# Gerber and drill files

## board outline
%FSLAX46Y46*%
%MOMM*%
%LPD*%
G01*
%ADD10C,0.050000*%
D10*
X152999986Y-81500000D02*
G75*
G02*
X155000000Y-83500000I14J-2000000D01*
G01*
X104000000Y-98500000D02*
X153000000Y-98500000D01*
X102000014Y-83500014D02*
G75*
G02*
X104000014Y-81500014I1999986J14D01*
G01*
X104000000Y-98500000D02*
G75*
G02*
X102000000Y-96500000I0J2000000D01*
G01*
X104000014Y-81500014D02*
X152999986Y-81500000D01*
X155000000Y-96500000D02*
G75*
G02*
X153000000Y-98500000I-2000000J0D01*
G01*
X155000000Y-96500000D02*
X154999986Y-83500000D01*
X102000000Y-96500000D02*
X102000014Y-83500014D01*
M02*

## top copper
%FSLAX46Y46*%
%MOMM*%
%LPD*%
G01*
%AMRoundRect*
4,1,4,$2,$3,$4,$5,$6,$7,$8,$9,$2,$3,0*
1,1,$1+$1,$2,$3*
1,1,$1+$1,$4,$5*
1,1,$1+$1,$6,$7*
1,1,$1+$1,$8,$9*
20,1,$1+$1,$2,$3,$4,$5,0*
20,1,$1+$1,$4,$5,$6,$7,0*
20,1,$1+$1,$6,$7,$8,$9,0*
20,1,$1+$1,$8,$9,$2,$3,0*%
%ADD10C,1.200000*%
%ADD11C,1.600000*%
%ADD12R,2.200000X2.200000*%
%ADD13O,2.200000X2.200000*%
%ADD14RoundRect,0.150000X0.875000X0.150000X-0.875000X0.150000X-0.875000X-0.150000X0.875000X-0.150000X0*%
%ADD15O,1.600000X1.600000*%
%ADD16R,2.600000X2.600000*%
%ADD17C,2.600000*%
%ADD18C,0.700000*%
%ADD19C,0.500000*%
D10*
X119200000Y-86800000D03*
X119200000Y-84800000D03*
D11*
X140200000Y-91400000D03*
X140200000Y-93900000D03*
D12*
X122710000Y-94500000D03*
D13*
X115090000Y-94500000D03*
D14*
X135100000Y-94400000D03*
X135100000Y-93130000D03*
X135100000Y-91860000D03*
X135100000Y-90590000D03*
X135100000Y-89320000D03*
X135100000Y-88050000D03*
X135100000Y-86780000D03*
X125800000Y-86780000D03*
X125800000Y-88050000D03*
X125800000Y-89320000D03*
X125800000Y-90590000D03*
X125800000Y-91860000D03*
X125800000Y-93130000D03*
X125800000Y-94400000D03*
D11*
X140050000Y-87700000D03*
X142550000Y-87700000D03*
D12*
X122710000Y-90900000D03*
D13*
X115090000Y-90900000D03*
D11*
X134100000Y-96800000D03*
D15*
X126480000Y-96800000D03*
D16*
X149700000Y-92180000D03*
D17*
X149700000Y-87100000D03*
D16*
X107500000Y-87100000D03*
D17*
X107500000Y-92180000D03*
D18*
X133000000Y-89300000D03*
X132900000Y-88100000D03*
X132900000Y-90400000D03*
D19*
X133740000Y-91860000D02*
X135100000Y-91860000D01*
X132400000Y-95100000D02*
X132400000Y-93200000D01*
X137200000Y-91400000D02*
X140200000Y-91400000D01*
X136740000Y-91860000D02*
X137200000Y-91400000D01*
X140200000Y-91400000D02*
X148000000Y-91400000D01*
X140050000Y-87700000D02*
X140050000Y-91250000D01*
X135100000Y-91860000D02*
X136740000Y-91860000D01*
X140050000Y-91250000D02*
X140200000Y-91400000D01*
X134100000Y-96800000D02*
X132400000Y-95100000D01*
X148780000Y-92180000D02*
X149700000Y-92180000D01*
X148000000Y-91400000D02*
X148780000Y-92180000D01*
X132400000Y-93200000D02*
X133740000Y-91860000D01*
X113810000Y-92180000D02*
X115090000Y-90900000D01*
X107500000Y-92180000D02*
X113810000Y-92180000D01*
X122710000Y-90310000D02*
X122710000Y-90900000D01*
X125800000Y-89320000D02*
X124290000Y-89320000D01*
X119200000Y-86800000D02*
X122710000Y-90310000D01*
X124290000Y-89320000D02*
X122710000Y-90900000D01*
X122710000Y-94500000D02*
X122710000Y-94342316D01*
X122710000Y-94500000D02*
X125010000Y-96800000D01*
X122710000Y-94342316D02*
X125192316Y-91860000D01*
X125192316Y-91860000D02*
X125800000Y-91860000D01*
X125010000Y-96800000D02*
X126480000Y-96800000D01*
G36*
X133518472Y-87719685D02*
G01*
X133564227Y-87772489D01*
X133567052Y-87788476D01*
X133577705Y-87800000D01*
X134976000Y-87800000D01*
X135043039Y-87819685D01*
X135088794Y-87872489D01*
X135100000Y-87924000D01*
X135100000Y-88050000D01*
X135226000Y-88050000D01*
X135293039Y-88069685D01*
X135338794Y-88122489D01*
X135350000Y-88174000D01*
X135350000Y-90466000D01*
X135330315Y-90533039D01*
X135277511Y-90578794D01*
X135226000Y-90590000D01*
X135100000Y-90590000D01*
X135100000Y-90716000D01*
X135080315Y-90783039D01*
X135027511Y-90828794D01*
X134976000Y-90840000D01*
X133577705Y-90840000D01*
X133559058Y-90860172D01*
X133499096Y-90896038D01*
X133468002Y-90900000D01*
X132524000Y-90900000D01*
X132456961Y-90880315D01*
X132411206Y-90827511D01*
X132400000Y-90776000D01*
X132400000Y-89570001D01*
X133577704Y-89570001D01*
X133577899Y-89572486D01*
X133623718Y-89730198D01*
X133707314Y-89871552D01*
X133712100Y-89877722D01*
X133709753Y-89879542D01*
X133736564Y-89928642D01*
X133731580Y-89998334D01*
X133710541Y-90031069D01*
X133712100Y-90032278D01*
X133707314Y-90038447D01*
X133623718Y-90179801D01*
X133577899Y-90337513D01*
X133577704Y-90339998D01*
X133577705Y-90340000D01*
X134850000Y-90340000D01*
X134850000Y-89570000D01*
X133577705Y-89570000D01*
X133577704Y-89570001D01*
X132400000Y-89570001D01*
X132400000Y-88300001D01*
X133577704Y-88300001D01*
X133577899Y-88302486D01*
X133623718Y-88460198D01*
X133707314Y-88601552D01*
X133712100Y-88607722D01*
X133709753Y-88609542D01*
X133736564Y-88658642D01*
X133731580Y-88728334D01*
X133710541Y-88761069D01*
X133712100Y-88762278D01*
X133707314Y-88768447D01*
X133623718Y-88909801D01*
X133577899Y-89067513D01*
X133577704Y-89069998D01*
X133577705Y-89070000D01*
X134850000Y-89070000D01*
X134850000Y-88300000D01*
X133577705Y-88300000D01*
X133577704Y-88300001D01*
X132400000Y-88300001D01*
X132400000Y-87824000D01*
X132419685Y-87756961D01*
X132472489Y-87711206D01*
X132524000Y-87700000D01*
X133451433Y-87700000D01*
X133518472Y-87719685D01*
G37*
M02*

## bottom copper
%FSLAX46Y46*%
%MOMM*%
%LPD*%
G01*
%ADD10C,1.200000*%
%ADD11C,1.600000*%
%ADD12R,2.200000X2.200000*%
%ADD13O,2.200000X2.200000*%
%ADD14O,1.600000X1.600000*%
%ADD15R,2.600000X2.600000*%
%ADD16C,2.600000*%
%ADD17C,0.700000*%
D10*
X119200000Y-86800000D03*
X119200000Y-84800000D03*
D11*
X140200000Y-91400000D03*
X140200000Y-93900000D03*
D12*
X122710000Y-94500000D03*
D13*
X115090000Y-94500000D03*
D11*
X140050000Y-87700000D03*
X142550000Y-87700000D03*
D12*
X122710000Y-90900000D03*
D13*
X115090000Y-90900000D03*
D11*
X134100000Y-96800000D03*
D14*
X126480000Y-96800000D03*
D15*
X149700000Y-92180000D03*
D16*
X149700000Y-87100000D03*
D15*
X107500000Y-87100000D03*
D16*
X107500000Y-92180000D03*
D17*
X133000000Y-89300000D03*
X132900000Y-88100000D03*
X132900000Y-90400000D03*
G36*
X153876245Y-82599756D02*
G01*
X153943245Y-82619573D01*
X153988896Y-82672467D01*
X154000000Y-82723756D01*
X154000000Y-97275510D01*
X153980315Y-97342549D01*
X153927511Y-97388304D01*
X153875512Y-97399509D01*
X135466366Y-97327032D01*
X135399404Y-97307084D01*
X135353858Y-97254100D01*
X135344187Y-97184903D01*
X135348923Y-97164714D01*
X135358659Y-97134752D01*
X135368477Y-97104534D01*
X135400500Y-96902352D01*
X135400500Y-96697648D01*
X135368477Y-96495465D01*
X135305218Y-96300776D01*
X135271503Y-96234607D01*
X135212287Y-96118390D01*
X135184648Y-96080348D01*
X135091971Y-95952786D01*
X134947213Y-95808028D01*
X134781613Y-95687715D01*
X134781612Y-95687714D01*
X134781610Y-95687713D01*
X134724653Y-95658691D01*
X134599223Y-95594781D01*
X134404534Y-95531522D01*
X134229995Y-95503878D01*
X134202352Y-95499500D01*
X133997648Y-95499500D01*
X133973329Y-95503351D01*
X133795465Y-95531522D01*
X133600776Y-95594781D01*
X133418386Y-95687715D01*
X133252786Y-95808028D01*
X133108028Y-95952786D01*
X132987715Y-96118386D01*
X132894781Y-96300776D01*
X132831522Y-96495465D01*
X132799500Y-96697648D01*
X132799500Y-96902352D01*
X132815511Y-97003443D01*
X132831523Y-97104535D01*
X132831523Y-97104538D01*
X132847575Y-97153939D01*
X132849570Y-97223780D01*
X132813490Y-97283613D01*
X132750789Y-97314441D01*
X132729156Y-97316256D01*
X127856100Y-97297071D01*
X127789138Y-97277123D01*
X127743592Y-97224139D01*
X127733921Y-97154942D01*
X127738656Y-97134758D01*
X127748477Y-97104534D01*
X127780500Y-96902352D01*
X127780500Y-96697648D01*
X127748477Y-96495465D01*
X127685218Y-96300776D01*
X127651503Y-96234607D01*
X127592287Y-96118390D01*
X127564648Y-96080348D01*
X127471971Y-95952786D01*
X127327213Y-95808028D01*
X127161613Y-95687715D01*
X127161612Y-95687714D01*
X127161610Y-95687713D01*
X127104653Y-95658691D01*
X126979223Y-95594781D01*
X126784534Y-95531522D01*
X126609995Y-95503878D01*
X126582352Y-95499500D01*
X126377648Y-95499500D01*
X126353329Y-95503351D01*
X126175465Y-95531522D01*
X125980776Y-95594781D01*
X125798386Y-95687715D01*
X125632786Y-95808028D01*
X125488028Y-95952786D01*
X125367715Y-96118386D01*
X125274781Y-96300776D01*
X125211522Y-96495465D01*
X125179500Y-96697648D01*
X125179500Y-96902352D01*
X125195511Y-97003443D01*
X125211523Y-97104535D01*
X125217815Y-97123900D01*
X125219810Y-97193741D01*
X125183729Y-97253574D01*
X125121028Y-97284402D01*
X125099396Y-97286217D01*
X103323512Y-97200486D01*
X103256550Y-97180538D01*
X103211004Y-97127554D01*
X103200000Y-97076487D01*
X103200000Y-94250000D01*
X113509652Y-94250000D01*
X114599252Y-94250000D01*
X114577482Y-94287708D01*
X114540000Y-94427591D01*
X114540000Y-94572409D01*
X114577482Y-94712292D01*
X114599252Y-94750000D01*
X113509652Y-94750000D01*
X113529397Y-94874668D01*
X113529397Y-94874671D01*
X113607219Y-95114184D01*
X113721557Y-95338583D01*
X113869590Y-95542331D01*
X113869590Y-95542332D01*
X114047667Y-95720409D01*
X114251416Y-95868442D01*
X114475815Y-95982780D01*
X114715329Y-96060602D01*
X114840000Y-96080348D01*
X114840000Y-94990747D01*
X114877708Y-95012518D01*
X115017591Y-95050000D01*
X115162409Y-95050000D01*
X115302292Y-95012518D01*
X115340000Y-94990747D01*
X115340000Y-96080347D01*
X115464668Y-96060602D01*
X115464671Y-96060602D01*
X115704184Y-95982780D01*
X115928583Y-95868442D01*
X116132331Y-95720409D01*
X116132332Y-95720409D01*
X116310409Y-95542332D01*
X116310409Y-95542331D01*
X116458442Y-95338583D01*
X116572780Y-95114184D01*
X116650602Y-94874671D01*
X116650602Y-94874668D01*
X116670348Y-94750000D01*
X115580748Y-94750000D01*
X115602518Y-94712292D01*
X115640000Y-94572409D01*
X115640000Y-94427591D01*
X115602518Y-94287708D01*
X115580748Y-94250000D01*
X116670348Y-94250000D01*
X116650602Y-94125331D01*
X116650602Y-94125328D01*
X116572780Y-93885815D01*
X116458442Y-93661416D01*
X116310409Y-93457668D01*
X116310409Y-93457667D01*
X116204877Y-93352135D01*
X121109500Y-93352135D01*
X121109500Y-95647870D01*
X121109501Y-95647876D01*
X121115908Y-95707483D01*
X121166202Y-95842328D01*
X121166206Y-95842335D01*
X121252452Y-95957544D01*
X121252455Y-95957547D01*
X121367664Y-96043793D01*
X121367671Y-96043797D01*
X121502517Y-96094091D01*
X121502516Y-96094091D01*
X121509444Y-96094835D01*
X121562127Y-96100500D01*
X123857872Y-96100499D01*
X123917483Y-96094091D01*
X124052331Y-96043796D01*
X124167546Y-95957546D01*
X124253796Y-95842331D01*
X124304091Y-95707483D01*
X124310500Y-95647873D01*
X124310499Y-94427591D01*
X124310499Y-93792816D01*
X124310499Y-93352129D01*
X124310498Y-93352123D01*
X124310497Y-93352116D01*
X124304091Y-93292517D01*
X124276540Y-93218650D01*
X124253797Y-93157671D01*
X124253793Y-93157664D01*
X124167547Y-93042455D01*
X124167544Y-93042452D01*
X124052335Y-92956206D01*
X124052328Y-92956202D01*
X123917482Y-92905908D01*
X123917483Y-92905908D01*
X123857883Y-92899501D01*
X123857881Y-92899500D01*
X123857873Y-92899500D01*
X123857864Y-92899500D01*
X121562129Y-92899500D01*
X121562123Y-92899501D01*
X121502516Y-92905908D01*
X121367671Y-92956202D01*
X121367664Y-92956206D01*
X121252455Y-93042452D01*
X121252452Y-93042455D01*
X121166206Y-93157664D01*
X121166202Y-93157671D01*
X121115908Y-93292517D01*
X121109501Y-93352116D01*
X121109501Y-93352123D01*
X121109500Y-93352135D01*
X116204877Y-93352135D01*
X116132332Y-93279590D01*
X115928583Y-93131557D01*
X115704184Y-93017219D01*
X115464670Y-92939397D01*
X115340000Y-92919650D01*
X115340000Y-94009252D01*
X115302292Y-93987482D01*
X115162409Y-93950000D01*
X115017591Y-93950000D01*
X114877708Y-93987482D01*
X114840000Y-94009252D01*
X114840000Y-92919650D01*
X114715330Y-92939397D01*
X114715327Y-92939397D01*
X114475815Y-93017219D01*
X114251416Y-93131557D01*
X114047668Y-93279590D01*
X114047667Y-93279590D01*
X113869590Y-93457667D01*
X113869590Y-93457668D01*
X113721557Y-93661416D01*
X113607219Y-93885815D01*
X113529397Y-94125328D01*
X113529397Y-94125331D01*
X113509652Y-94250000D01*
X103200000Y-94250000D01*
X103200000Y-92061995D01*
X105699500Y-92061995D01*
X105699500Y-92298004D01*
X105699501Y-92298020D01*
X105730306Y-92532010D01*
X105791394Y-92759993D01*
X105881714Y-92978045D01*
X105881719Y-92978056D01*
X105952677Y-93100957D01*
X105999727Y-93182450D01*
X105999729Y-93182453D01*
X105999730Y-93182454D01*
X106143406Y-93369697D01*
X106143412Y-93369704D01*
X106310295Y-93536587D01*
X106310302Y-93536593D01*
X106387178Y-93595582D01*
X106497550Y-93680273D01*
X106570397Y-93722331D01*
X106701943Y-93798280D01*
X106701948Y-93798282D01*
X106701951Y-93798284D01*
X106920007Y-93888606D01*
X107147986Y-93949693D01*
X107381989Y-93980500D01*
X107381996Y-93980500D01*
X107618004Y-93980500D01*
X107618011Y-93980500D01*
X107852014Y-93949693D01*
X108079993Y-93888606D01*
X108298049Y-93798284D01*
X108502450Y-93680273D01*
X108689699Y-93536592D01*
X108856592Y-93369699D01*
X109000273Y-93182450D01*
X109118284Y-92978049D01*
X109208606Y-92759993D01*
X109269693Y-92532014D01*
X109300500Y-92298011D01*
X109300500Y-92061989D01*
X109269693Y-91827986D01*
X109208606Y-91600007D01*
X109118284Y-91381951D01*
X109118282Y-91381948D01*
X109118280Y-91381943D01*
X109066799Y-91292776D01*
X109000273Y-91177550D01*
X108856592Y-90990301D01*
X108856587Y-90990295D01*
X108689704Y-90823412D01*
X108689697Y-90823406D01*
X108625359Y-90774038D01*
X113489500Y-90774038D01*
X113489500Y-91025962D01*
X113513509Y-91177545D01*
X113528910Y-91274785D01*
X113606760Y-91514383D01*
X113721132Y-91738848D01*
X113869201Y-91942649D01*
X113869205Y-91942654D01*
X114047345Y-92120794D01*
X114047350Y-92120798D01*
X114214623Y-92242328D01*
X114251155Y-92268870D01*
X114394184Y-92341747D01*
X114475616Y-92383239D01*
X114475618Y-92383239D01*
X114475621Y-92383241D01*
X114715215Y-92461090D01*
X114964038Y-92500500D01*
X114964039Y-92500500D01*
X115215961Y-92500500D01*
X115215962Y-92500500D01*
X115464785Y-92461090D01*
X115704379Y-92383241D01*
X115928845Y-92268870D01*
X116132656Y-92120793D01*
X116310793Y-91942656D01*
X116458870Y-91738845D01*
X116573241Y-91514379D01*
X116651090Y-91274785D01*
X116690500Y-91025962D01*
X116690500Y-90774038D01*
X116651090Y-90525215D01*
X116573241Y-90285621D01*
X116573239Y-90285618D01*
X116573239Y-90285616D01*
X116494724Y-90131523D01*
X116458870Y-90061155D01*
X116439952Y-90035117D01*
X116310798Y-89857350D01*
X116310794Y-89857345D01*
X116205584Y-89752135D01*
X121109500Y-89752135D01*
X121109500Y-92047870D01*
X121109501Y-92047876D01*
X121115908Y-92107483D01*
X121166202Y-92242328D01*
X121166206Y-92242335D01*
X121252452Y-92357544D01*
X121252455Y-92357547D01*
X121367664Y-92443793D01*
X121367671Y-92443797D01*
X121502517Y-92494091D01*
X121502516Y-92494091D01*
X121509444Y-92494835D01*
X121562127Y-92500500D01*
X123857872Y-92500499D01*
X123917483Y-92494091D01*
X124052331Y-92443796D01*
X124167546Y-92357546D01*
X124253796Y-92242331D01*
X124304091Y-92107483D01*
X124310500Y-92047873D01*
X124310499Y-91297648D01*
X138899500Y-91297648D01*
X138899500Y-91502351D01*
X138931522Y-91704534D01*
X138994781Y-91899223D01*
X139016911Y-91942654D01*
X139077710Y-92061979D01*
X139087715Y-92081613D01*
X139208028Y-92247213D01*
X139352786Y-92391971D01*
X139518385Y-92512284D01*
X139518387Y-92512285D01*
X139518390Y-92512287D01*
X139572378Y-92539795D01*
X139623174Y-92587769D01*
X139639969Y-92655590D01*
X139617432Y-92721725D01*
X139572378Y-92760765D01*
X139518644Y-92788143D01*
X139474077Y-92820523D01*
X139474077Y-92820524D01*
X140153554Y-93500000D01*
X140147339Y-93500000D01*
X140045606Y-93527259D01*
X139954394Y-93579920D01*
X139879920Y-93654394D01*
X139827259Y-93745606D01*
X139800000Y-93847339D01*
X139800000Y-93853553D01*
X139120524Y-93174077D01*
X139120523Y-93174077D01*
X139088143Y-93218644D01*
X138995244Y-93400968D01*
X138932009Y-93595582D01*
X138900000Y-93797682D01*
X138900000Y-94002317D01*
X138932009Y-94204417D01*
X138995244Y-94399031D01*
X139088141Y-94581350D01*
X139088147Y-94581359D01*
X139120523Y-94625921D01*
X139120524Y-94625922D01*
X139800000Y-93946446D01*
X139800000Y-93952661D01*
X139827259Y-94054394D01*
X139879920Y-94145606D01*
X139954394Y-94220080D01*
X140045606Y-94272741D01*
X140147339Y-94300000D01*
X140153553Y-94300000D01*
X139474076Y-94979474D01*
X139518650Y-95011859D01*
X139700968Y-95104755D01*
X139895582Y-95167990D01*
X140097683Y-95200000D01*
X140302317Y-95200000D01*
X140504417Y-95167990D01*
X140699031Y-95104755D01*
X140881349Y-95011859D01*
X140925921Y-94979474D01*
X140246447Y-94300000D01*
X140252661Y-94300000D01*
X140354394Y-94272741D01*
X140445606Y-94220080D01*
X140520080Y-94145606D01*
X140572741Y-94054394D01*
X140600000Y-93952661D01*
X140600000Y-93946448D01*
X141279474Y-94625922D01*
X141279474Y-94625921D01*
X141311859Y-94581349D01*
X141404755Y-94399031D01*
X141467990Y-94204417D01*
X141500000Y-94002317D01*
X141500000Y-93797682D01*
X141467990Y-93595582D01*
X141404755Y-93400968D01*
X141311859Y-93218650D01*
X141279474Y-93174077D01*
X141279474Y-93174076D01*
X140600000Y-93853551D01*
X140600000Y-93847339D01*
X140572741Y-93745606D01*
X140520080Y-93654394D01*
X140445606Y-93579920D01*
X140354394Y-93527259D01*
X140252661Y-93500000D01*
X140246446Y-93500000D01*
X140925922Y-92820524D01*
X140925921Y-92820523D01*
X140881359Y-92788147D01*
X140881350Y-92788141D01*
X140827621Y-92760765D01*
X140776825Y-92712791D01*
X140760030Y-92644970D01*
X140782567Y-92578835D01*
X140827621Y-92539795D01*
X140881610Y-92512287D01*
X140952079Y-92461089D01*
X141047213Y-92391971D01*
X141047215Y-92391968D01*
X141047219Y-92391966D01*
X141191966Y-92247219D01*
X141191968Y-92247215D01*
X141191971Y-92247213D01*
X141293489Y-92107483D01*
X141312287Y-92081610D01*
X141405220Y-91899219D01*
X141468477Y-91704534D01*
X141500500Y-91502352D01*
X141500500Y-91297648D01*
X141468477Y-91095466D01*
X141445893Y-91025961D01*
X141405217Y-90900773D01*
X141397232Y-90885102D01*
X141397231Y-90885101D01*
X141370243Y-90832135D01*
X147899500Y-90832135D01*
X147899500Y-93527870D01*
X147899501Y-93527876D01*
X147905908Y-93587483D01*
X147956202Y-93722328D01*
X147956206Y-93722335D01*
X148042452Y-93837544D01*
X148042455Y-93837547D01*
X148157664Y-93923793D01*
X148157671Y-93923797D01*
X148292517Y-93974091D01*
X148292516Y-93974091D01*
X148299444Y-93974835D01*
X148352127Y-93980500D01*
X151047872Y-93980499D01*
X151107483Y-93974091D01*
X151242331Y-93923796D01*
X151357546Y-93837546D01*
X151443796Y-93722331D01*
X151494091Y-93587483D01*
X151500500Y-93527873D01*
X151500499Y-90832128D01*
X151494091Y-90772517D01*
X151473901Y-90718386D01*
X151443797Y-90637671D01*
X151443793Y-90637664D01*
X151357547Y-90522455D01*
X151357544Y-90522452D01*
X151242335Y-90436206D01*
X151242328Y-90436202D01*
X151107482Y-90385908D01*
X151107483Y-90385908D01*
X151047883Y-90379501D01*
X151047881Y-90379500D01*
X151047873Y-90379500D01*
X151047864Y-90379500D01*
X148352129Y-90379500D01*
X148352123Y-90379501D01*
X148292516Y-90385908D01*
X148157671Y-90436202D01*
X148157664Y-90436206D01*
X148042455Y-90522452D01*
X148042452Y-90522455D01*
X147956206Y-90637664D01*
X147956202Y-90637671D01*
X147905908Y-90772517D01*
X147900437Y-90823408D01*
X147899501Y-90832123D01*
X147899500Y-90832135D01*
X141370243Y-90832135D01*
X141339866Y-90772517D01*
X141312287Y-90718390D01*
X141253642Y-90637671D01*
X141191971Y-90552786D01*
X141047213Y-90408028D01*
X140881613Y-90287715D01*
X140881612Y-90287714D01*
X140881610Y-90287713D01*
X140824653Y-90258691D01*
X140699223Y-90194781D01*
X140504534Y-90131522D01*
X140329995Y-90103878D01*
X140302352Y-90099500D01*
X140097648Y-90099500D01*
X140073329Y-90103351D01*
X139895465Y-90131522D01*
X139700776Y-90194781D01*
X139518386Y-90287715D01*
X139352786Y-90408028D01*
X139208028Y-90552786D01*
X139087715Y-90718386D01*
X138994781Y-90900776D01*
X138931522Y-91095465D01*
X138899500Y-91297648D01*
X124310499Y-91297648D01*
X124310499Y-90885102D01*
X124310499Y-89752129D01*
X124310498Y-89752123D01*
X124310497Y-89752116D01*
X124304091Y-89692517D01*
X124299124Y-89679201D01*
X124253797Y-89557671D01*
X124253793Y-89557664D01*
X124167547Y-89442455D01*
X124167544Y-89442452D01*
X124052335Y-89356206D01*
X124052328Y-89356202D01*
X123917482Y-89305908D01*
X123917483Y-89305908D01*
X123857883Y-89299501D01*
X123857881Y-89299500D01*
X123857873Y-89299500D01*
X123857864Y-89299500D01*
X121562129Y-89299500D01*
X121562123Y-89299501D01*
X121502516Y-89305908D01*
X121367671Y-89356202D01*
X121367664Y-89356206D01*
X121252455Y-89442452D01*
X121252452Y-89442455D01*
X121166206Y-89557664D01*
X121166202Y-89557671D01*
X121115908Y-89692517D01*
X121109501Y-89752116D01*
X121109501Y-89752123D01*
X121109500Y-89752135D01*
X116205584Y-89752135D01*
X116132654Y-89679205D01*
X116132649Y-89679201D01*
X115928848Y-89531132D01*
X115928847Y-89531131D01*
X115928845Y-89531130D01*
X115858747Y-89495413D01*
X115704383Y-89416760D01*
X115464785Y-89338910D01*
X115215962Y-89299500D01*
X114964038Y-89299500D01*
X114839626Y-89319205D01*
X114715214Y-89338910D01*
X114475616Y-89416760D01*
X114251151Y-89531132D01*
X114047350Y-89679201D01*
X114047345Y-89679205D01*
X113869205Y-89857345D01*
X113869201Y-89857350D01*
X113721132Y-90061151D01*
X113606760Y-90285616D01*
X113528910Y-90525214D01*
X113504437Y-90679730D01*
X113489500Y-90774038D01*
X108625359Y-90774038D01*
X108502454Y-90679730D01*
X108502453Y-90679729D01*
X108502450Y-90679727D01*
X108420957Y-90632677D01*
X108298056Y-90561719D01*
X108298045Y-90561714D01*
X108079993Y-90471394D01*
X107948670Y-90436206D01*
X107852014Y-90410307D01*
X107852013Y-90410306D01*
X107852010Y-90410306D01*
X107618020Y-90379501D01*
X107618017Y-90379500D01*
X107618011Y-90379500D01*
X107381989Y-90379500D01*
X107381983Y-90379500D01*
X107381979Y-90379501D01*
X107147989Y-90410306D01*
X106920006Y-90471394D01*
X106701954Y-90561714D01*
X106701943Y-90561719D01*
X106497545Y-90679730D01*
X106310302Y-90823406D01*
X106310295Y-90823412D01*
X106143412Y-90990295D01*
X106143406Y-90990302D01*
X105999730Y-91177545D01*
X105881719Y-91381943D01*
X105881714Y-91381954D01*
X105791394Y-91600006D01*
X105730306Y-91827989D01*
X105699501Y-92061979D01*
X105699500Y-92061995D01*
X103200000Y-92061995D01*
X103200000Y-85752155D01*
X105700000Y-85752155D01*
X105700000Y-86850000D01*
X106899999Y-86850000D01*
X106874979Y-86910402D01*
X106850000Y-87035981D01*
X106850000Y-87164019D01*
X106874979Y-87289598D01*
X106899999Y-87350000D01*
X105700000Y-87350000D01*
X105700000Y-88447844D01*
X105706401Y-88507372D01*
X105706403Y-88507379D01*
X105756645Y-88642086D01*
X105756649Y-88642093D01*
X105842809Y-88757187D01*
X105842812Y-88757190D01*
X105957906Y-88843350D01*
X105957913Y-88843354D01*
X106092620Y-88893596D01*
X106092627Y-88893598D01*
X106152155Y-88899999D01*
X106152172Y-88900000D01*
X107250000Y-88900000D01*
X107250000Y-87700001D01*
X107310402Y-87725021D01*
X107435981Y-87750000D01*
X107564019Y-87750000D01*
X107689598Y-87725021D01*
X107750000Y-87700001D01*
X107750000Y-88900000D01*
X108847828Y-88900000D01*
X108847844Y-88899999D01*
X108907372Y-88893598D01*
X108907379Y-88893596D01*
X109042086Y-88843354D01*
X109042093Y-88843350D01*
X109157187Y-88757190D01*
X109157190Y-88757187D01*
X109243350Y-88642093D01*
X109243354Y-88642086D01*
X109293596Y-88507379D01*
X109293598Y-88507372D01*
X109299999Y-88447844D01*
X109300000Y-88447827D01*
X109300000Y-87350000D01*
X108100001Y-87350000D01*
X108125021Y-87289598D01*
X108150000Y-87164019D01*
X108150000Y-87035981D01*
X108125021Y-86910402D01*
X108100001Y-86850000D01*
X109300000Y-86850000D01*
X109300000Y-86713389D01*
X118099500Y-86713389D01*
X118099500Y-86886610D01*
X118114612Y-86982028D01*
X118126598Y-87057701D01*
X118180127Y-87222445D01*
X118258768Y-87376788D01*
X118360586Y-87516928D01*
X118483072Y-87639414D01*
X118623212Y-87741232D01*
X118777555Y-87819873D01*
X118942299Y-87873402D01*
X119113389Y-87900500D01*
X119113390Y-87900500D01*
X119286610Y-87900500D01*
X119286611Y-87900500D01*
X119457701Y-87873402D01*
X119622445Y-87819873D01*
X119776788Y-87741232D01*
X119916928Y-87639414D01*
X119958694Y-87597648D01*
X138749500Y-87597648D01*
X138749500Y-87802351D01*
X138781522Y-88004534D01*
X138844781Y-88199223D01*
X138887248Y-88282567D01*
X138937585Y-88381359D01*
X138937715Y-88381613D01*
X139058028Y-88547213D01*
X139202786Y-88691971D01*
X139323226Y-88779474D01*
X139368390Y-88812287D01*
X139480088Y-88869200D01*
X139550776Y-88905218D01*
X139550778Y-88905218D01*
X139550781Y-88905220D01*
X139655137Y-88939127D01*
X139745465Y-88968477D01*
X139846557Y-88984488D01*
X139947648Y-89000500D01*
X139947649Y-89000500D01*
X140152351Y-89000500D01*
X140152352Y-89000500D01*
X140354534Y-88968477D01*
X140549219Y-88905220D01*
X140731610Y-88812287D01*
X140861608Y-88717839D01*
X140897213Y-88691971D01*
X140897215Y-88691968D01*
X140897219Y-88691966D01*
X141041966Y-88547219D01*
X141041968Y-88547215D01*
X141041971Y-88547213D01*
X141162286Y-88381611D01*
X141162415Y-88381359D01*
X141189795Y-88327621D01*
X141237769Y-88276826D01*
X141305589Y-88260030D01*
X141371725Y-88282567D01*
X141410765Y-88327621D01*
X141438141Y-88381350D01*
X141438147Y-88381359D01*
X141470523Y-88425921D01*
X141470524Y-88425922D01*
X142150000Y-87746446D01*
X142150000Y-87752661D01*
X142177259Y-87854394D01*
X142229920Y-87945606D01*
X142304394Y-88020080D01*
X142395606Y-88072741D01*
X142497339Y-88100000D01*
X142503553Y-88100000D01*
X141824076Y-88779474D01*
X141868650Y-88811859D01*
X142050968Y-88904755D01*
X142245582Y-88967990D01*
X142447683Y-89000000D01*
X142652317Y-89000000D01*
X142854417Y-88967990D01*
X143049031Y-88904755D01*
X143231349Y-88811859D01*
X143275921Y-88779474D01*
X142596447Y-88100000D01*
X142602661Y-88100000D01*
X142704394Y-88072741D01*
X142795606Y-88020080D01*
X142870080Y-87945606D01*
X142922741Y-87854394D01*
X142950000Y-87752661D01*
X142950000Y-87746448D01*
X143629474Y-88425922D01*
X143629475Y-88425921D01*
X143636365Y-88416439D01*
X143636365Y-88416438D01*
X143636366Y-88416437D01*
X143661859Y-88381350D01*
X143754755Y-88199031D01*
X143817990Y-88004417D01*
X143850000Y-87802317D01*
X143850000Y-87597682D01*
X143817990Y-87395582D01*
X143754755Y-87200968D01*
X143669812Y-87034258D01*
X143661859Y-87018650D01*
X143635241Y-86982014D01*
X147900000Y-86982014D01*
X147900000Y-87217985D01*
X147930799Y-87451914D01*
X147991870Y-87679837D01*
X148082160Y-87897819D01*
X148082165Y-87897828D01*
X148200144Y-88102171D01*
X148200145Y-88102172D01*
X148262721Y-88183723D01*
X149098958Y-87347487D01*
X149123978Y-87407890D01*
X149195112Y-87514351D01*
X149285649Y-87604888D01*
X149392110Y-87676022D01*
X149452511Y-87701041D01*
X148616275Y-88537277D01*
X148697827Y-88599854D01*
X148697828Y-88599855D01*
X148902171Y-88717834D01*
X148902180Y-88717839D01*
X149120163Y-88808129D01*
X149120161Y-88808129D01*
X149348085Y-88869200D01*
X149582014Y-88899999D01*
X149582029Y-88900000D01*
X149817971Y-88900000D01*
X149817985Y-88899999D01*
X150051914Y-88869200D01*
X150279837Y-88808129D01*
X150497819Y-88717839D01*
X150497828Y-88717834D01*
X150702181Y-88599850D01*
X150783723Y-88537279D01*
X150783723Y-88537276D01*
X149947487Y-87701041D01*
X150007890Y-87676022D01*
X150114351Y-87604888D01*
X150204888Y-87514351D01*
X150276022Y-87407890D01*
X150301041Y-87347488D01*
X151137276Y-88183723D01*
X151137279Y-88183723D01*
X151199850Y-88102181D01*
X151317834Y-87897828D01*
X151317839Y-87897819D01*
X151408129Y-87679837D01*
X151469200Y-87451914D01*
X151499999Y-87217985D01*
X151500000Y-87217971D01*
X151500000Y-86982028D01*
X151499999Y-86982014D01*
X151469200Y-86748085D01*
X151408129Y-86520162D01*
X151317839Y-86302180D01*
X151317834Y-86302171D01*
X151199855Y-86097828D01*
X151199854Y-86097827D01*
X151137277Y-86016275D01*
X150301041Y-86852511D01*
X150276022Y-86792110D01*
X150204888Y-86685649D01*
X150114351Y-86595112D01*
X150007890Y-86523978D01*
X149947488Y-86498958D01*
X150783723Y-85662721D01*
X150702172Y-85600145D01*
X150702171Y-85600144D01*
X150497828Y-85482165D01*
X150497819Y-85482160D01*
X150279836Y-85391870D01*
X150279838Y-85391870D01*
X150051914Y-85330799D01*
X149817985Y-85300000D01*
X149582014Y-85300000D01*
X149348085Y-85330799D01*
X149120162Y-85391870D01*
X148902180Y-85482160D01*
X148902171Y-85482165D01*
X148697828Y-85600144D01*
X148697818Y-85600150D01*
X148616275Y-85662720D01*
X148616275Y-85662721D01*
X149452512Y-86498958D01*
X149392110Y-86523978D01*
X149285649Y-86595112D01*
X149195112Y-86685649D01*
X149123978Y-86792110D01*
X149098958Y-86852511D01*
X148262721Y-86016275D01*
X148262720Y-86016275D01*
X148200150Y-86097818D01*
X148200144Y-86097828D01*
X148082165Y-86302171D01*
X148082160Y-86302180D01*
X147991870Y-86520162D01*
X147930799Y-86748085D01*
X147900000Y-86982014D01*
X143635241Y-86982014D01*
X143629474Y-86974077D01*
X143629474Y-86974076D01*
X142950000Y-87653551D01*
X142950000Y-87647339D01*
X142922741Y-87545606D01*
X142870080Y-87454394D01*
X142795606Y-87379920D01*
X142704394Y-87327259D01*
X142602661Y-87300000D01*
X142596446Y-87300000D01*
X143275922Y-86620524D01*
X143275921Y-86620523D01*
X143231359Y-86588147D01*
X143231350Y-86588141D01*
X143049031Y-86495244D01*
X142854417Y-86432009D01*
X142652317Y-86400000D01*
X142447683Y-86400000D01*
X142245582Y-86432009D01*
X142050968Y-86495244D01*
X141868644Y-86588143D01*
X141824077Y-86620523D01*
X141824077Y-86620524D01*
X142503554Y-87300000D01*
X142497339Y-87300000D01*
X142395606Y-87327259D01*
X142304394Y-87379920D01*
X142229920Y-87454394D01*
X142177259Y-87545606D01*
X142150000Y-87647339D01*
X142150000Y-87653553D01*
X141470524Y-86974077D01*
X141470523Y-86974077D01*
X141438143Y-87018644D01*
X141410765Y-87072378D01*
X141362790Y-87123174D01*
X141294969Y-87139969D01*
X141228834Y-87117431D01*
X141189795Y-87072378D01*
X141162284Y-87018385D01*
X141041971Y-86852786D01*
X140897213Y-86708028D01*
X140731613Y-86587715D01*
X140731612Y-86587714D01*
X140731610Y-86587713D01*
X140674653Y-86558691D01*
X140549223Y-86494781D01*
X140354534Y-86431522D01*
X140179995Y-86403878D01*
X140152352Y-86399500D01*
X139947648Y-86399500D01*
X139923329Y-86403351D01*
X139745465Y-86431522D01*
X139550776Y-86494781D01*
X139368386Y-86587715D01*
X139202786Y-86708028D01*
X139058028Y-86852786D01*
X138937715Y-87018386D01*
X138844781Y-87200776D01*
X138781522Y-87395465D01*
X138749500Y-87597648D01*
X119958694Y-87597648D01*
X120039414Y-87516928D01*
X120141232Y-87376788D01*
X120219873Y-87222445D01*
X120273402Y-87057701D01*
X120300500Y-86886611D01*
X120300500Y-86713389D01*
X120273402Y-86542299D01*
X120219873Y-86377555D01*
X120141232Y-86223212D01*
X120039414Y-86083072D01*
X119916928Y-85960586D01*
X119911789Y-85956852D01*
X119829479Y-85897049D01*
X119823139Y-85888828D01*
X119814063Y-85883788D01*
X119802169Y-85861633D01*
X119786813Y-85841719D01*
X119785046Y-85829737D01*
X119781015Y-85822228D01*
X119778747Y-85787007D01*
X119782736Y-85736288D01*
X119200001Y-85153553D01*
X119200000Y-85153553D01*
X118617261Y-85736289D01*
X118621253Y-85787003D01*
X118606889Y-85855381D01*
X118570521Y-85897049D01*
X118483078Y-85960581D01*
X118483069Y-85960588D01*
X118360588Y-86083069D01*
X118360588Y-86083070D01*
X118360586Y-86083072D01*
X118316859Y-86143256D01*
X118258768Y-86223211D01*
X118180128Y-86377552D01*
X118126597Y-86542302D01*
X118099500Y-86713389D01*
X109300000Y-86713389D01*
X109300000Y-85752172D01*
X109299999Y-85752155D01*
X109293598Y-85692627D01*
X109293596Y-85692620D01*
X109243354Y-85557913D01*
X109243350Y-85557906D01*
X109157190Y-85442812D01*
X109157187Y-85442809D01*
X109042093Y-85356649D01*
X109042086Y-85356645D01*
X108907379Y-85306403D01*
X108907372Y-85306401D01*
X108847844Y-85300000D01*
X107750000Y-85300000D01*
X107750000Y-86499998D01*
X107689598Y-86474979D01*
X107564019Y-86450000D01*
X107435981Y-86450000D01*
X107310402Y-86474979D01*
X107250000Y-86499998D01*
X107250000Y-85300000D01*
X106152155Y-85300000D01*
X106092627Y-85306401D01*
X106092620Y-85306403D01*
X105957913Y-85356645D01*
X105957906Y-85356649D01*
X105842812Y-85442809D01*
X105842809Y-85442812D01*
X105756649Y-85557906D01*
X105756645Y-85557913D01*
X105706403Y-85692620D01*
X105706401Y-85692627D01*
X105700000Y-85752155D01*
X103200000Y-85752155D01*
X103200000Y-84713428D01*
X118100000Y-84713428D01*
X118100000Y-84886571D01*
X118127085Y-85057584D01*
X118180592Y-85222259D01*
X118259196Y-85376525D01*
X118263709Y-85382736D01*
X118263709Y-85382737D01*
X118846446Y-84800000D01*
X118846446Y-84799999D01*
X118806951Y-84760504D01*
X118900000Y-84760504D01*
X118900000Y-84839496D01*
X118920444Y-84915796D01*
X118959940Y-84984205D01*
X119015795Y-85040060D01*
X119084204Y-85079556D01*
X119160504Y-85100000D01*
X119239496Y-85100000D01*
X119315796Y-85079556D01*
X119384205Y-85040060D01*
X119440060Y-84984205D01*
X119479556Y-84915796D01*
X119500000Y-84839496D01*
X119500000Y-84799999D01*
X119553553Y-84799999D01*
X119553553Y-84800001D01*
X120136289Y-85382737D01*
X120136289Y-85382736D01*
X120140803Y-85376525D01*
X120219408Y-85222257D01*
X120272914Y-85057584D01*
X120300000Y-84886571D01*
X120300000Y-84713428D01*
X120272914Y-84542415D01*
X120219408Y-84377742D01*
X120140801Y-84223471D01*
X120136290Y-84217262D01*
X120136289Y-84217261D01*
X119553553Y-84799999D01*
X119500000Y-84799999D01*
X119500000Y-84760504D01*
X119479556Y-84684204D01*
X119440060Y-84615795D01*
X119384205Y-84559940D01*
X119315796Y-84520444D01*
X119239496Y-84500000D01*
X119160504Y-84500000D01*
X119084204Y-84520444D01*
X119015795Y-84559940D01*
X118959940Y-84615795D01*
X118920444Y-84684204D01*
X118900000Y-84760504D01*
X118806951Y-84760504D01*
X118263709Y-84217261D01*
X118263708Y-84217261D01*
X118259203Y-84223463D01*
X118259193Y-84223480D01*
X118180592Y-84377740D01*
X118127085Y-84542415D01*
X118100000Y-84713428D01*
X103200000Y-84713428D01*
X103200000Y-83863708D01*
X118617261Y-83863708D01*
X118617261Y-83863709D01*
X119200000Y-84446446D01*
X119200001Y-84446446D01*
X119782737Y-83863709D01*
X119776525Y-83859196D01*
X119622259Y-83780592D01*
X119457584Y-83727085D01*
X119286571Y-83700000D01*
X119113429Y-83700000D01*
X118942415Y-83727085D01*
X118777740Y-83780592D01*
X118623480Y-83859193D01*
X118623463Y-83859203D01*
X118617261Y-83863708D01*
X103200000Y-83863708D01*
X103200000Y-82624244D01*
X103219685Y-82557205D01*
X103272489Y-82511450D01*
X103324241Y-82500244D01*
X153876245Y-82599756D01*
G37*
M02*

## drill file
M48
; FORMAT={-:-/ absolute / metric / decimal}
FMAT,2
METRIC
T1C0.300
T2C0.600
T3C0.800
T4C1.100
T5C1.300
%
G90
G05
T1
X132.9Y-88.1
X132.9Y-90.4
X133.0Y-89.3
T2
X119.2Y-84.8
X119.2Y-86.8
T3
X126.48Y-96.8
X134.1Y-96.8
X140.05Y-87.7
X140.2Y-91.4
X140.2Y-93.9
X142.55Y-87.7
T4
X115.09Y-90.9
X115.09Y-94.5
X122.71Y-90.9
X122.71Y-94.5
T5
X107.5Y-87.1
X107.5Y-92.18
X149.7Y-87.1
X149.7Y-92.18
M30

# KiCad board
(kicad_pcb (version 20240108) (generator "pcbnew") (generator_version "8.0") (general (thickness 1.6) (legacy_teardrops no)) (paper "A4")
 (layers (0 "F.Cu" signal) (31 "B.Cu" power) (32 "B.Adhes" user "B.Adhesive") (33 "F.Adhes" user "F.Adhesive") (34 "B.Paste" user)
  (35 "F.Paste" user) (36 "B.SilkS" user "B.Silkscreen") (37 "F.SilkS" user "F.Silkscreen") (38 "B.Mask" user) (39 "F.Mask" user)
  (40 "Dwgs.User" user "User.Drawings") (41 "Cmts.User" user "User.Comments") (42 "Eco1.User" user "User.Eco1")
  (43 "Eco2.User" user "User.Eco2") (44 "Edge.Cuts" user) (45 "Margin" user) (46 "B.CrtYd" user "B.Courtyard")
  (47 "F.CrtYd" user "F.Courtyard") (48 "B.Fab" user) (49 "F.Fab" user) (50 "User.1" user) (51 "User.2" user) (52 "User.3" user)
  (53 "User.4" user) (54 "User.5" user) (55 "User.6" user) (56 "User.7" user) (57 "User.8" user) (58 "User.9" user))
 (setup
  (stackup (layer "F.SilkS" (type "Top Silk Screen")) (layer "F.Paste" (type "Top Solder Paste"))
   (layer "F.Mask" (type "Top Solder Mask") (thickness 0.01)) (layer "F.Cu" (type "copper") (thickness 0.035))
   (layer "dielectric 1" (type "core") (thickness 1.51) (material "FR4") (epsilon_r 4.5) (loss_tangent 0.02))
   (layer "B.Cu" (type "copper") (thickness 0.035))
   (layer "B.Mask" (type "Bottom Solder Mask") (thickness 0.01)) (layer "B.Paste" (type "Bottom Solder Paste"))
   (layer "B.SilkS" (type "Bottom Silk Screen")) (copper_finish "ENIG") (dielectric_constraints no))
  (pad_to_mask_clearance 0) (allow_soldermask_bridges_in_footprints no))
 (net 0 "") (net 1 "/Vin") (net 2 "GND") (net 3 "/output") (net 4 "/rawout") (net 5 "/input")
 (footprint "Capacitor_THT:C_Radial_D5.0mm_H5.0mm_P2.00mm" (layer "F.Cu") (at 119.2 86.8 90)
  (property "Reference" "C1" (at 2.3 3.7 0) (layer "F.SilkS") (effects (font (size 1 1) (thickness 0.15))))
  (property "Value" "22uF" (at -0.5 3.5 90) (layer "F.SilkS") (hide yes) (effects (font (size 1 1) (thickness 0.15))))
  (pad "1" thru_hole circle (at 0 0 90) (size 1.2 1.2) (drill 0.6) (layers "*.Cu" "*.Mask") (remove_unused_layers no) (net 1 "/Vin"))
  (pad "2" thru_hole circle (at 2 0 90) (size 1.2 1.2) (drill 0.6) (layers "*.Cu" "*.Mask") (remove_unused_layers no) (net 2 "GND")))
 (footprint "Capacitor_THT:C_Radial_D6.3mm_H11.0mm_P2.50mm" (layer "F.Cu") (at 140.2 91.4 -90)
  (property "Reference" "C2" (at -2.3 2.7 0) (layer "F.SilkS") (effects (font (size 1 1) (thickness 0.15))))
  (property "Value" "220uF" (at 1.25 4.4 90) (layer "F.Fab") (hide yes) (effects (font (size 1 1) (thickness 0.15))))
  (pad "1" thru_hole circle (at 0 0 270) (size 1.6 1.6) (drill 0.8) (layers "*.Cu" "*.Mask") (remove_unused_layers no) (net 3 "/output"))
  (pad "2" thru_hole circle (at 2.5 0 270) (size 1.6 1.6) (drill 0.8) (layers "*.Cu" "*.Mask") (remove_unused_layers no) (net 2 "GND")))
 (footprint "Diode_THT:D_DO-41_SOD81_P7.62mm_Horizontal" (layer "F.Cu") (at 122.71 94.5 180)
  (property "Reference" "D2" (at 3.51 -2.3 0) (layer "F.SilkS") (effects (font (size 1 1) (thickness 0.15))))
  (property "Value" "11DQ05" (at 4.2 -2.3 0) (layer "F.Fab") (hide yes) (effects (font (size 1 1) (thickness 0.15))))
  (pad "1" thru_hole rect (at 0 0 180) (size 2.2 2.2) (drill 1.1) (layers "*.Cu" "*.Mask") (remove_unused_layers no) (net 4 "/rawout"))
  (pad "2" thru_hole oval (at 7.62 0 180) (size 2.2 2.2) (drill 1.1) (layers "*.Cu" "*.Mask") (remove_unused_layers no) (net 2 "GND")))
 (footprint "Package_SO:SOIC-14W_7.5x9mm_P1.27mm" (layer "F.Cu") (at 130.45 90.59 180)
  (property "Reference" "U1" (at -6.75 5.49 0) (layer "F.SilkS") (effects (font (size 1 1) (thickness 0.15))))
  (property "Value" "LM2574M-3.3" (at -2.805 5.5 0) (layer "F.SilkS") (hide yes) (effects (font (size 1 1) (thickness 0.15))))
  (pad "1" smd roundrect (at -4.65 -3.81 180) (size 2.05 0.6) (layers "F.Cu" "F.Paste" "F.Mask") (roundrect_rratio 0.25))
  (pad "2" smd roundrect (at -4.65 -2.54 180) (size 2.05 0.6) (layers "F.Cu" "F.Paste" "F.Mask") (roundrect_rratio 0.25))
  (pad "3" smd roundrect (at -4.65 -1.27 180) (size 2.05 0.6) (layers "F.Cu" "F.Paste" "F.Mask") (roundrect_rratio 0.25) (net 3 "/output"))
  (pad "4" smd roundrect (at -4.65 0 180) (size 2.05 0.6) (layers "F.Cu" "F.Paste" "F.Mask") (roundrect_rratio 0.25) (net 2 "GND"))
  (pad "5" smd roundrect (at -4.65 1.27 180) (size 2.05 0.6) (layers "F.Cu" "F.Paste" "F.Mask") (roundrect_rratio 0.25) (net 2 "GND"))
  (pad "6" smd roundrect (at -4.65 2.54 180) (size 2.05 0.6) (layers "F.Cu" "F.Paste" "F.Mask") (roundrect_rratio 0.25) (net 2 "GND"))
  (pad "7" smd roundrect (at -4.65 3.81 180) (size 2.05 0.6) (layers "F.Cu" "F.Paste" "F.Mask") (roundrect_rratio 0.25))
  (pad "8" smd roundrect (at 4.65 3.81 180) (size 2.05 0.6) (layers "F.Cu" "F.Paste" "F.Mask") (roundrect_rratio 0.25))
  (pad "9" smd roundrect (at 4.65 2.54 180) (size 2.05 0.6) (layers "F.Cu" "F.Paste" "F.Mask") (roundrect_rratio 0.25))
  (pad "10" smd roundrect (at 4.65 1.27 180) (size 2.05 0.6) (layers "F.Cu" "F.Paste" "F.Mask") (roundrect_rratio 0.25) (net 1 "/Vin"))
  (pad "11" smd roundrect (at 4.65 0 180) (size 2.05 0.6) (layers "F.Cu" "F.Paste" "F.Mask") (roundrect_rratio 0.25))
  (pad "12" smd roundrect (at 4.65 -1.27 180) (size 2.05 0.6) (layers "F.Cu" "F.Paste" "F.Mask") (roundrect_rratio 0.25) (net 4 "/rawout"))
  (pad "13" smd roundrect (at 4.65 -2.54 180) (size 2.05 0.6) (layers "F.Cu" "F.Paste" "F.Mask") (roundrect_rratio 0.25))
  (pad "14" smd roundrect (at 4.65 -3.81 180) (size 2.05 0.6) (layers "F.Cu" "F.Paste" "F.Mask") (roundrect_rratio 0.25)))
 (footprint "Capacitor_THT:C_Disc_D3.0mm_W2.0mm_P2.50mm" (layer "F.Cu") (at 140.05 87.7)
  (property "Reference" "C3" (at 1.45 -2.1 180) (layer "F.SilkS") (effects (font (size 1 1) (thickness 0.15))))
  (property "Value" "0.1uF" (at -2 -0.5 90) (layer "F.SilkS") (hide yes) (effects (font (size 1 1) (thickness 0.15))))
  (pad "1" thru_hole circle (at 0 0) (size 1.6 1.6) (drill 0.8) (layers "*.Cu" "*.Mask") (remove_unused_layers no) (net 3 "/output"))
  (pad "2" thru_hole circle (at 2.5 0) (size 1.6 1.6) (drill 0.8) (layers "*.Cu" "*.Mask") (remove_unused_layers no) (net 2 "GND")))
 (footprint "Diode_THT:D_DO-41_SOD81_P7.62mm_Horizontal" (layer "F.Cu") (at 122.71 90.9 180)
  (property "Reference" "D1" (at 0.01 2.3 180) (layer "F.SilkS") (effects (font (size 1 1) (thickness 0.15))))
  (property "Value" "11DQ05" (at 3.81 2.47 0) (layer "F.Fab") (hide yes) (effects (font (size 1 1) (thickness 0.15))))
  (pad "1" thru_hole rect (at 0 0 180) (size 2.2 2.2) (drill 1.1) (layers "*.Cu" "*.Mask") (remove_unused_layers no) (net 1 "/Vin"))
  (pad "2" thru_hole oval (at 7.62 0 180) (size 2.2 2.2) (drill 1.1) (layers "*.Cu" "*.Mask") (remove_unused_layers no) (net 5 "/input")))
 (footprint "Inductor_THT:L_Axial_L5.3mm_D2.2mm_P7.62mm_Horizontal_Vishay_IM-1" (layer "F.Cu") (at 134.1 96.8 180)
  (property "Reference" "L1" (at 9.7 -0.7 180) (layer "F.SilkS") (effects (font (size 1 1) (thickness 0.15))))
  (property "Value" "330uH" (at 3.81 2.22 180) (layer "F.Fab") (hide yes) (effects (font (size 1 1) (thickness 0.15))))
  (pad "1" thru_hole circle (at 0 0 180) (size 1.6 1.6) (drill 0.8) (layers "*.Cu" "*.Mask") (remove_unused_layers no) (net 3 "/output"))
  (pad "2" thru_hole oval (at 7.62 0 180) (size 1.6 1.6) (drill 0.8) (layers "*.Cu" "*.Mask") (remove_unused_layers no) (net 4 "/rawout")))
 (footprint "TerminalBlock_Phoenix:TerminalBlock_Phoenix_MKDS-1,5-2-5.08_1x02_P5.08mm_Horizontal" (layer "F.Cu") (at 149.7 92.18 90)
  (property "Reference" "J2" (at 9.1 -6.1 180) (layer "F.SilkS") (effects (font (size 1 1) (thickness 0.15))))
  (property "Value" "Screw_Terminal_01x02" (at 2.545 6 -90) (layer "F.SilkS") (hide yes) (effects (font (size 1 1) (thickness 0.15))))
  (pad "1" thru_hole rect (at 0 0 90) (size 2.6 2.6) (drill 1.3) (layers "*.Cu" "*.Mask") (remove_unused_layers no) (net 3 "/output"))
  (pad "2" thru_hole circle (at 5.08 0 90) (size 2.6 2.6) (drill 1.3) (layers "*.Cu" "*.Mask") (remove_unused_layers no) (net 2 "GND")))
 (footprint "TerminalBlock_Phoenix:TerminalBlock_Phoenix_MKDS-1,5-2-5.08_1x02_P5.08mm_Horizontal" (layer "F.Cu") (at 107.5 87.1 -90)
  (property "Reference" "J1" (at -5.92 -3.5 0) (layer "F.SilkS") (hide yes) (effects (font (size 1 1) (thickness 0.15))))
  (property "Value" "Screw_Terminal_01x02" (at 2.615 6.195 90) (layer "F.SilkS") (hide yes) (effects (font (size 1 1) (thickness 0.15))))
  (pad "1" thru_hole rect (at 0 0 270) (size 2.6 2.6) (drill 1.3) (layers "*.Cu" "*.Mask") (remove_unused_layers no) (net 2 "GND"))
  (pad "2" thru_hole circle (at 5.08 0 270) (size 2.6 2.6) (drill 1.3) (layers "*.Cu" "*.Mask") (remove_unused_layers no) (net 5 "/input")))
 (gr_arc (start 152.999986 81.5) (mid 154.414209 82.085781) (end 154.999986 83.5) (stroke (width 0.05) (type default)) (layer "Edge.Cuts"))
 (gr_line (start 104 98.5) (end 153 98.5) (stroke (width 0.05) (type default)) (layer "Edge.Cuts"))
 (gr_arc (start 102.000014 83.500014) (mid 102.585796 82.085796) (end 104.000014 81.500014) (stroke (width 0.05) (type default))
  (layer "Edge.Cuts"))
 (gr_arc (start 104 98.5) (mid 102.585786 97.914214) (end 102 96.5) (stroke (width 0.05) (type default)) (layer "Edge.Cuts"))
 (gr_line (start 104.000014 81.500014) (end 152.999986 81.5) (stroke (width 0.05) (type default)) (layer "Edge.Cuts"))
 (gr_arc (start 155 96.5) (mid 154.414214 97.914214) (end 153 98.5) (stroke (width 0.05) (type default)) (layer "Edge.Cuts"))
 (gr_line (start 155 96.5) (end 154.999986 83.5) (stroke (width 0.05) (type default)) (layer "Edge.Cuts"))
 (gr_line (start 102 96.5) (end 102.000014 83.500014) (stroke (width 0.05) (type default)) (layer "Edge.Cuts"))
 (via (at 133 89.3) (size 0.7) (drill 0.3) (layers "F.Cu" "B.Cu") (free yes) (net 2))
 (via (at 132.9 88.1) (size 0.7) (drill 0.3) (layers "F.Cu" "B.Cu") (free yes) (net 2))
 (via (at 132.9 90.4) (size 0.7) (drill 0.3) (layers "F.Cu" "B.Cu") (free yes) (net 2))
 (segment (start 133.74 91.86) (end 135.1 91.86) (width 0.5) (layer "F.Cu") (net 3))
 (segment (start 132.4 95.1) (end 132.4 93.2) (width 0.5) (layer "F.Cu") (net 3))
 (segment (start 137.2 91.4) (end 140.2 91.4) (width 0.5) (layer "F.Cu") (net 3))
 (segment (start 136.74 91.86) (end 137.2 91.4) (width 0.5) (layer "F.Cu") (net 3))
 (segment (start 140.2 91.4) (end 148 91.4) (width 0.5) (layer "F.Cu") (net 3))
 (segment (start 140.05 87.7) (end 140.05 91.25) (width 0.5) (layer "F.Cu") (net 3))
 (segment (start 135.1 91.86) (end 136.74 91.86) (width 0.5) (layer "F.Cu") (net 3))
 (segment (start 140.05 91.25) (end 140.2 91.4) (width 0.5) (layer "F.Cu") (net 3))
 (segment (start 134.1 96.8) (end 132.4 95.1) (width 0.5) (layer "F.Cu") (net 3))
 (segment (start 148.78 92.18) (end 149.7 92.18) (width 0.5) (layer "F.Cu") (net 3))
 (segment (start 148 91.4) (end 148.78 92.18) (width 0.5) (layer "F.Cu") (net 3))
 (segment (start 132.4 93.2) (end 133.74 91.86) (width 0.5) (layer "F.Cu") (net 3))
 (segment (start 113.81 92.18) (end 115.09 90.9) (width 0.5) (layer "F.Cu") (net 5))
 (segment (start 107.5 92.18) (end 113.81 92.18) (width 0.5) (layer "F.Cu") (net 5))
 (segment (start 122.71 90.31) (end 122.71 90.9) (width 0.5) (layer "F.Cu") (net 1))
 (segment (start 125.8 89.32) (end 124.29 89.32) (width 0.5) (layer "F.Cu") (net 1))
 (segment (start 119.2 86.8) (end 122.71 90.31) (width 0.5) (layer "F.Cu") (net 1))
 (segment (start 124.29 89.32) (end 122.71 90.9) (width 0.5) (layer "F.Cu") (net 1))
 (segment (start 122.71 94.5) (end 122.71 94.342316) (width 0.5) (layer "F.Cu") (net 4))
 (segment (start 122.71 94.5) (end 125.01 96.8) (width 0.5) (layer "F.Cu") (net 4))
 (segment (start 122.71 94.342316) (end 125.192316 91.86) (width 0.5) (layer "F.Cu") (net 4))
 (segment (start 125.192316 91.86) (end 125.8 91.86) (width 0.5) (layer "F.Cu") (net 4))
 (segment (start 125.01 96.8) (end 126.48 96.8) (width 0.5) (layer "F.Cu") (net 4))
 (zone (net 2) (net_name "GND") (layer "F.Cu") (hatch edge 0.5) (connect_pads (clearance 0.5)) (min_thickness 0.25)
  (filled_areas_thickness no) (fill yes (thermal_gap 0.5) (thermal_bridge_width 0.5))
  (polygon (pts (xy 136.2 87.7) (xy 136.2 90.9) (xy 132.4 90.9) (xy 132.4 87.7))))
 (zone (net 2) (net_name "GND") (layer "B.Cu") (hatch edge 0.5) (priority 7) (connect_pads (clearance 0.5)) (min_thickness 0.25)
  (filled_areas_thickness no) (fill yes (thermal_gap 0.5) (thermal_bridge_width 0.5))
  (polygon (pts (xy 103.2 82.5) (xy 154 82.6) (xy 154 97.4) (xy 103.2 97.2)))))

